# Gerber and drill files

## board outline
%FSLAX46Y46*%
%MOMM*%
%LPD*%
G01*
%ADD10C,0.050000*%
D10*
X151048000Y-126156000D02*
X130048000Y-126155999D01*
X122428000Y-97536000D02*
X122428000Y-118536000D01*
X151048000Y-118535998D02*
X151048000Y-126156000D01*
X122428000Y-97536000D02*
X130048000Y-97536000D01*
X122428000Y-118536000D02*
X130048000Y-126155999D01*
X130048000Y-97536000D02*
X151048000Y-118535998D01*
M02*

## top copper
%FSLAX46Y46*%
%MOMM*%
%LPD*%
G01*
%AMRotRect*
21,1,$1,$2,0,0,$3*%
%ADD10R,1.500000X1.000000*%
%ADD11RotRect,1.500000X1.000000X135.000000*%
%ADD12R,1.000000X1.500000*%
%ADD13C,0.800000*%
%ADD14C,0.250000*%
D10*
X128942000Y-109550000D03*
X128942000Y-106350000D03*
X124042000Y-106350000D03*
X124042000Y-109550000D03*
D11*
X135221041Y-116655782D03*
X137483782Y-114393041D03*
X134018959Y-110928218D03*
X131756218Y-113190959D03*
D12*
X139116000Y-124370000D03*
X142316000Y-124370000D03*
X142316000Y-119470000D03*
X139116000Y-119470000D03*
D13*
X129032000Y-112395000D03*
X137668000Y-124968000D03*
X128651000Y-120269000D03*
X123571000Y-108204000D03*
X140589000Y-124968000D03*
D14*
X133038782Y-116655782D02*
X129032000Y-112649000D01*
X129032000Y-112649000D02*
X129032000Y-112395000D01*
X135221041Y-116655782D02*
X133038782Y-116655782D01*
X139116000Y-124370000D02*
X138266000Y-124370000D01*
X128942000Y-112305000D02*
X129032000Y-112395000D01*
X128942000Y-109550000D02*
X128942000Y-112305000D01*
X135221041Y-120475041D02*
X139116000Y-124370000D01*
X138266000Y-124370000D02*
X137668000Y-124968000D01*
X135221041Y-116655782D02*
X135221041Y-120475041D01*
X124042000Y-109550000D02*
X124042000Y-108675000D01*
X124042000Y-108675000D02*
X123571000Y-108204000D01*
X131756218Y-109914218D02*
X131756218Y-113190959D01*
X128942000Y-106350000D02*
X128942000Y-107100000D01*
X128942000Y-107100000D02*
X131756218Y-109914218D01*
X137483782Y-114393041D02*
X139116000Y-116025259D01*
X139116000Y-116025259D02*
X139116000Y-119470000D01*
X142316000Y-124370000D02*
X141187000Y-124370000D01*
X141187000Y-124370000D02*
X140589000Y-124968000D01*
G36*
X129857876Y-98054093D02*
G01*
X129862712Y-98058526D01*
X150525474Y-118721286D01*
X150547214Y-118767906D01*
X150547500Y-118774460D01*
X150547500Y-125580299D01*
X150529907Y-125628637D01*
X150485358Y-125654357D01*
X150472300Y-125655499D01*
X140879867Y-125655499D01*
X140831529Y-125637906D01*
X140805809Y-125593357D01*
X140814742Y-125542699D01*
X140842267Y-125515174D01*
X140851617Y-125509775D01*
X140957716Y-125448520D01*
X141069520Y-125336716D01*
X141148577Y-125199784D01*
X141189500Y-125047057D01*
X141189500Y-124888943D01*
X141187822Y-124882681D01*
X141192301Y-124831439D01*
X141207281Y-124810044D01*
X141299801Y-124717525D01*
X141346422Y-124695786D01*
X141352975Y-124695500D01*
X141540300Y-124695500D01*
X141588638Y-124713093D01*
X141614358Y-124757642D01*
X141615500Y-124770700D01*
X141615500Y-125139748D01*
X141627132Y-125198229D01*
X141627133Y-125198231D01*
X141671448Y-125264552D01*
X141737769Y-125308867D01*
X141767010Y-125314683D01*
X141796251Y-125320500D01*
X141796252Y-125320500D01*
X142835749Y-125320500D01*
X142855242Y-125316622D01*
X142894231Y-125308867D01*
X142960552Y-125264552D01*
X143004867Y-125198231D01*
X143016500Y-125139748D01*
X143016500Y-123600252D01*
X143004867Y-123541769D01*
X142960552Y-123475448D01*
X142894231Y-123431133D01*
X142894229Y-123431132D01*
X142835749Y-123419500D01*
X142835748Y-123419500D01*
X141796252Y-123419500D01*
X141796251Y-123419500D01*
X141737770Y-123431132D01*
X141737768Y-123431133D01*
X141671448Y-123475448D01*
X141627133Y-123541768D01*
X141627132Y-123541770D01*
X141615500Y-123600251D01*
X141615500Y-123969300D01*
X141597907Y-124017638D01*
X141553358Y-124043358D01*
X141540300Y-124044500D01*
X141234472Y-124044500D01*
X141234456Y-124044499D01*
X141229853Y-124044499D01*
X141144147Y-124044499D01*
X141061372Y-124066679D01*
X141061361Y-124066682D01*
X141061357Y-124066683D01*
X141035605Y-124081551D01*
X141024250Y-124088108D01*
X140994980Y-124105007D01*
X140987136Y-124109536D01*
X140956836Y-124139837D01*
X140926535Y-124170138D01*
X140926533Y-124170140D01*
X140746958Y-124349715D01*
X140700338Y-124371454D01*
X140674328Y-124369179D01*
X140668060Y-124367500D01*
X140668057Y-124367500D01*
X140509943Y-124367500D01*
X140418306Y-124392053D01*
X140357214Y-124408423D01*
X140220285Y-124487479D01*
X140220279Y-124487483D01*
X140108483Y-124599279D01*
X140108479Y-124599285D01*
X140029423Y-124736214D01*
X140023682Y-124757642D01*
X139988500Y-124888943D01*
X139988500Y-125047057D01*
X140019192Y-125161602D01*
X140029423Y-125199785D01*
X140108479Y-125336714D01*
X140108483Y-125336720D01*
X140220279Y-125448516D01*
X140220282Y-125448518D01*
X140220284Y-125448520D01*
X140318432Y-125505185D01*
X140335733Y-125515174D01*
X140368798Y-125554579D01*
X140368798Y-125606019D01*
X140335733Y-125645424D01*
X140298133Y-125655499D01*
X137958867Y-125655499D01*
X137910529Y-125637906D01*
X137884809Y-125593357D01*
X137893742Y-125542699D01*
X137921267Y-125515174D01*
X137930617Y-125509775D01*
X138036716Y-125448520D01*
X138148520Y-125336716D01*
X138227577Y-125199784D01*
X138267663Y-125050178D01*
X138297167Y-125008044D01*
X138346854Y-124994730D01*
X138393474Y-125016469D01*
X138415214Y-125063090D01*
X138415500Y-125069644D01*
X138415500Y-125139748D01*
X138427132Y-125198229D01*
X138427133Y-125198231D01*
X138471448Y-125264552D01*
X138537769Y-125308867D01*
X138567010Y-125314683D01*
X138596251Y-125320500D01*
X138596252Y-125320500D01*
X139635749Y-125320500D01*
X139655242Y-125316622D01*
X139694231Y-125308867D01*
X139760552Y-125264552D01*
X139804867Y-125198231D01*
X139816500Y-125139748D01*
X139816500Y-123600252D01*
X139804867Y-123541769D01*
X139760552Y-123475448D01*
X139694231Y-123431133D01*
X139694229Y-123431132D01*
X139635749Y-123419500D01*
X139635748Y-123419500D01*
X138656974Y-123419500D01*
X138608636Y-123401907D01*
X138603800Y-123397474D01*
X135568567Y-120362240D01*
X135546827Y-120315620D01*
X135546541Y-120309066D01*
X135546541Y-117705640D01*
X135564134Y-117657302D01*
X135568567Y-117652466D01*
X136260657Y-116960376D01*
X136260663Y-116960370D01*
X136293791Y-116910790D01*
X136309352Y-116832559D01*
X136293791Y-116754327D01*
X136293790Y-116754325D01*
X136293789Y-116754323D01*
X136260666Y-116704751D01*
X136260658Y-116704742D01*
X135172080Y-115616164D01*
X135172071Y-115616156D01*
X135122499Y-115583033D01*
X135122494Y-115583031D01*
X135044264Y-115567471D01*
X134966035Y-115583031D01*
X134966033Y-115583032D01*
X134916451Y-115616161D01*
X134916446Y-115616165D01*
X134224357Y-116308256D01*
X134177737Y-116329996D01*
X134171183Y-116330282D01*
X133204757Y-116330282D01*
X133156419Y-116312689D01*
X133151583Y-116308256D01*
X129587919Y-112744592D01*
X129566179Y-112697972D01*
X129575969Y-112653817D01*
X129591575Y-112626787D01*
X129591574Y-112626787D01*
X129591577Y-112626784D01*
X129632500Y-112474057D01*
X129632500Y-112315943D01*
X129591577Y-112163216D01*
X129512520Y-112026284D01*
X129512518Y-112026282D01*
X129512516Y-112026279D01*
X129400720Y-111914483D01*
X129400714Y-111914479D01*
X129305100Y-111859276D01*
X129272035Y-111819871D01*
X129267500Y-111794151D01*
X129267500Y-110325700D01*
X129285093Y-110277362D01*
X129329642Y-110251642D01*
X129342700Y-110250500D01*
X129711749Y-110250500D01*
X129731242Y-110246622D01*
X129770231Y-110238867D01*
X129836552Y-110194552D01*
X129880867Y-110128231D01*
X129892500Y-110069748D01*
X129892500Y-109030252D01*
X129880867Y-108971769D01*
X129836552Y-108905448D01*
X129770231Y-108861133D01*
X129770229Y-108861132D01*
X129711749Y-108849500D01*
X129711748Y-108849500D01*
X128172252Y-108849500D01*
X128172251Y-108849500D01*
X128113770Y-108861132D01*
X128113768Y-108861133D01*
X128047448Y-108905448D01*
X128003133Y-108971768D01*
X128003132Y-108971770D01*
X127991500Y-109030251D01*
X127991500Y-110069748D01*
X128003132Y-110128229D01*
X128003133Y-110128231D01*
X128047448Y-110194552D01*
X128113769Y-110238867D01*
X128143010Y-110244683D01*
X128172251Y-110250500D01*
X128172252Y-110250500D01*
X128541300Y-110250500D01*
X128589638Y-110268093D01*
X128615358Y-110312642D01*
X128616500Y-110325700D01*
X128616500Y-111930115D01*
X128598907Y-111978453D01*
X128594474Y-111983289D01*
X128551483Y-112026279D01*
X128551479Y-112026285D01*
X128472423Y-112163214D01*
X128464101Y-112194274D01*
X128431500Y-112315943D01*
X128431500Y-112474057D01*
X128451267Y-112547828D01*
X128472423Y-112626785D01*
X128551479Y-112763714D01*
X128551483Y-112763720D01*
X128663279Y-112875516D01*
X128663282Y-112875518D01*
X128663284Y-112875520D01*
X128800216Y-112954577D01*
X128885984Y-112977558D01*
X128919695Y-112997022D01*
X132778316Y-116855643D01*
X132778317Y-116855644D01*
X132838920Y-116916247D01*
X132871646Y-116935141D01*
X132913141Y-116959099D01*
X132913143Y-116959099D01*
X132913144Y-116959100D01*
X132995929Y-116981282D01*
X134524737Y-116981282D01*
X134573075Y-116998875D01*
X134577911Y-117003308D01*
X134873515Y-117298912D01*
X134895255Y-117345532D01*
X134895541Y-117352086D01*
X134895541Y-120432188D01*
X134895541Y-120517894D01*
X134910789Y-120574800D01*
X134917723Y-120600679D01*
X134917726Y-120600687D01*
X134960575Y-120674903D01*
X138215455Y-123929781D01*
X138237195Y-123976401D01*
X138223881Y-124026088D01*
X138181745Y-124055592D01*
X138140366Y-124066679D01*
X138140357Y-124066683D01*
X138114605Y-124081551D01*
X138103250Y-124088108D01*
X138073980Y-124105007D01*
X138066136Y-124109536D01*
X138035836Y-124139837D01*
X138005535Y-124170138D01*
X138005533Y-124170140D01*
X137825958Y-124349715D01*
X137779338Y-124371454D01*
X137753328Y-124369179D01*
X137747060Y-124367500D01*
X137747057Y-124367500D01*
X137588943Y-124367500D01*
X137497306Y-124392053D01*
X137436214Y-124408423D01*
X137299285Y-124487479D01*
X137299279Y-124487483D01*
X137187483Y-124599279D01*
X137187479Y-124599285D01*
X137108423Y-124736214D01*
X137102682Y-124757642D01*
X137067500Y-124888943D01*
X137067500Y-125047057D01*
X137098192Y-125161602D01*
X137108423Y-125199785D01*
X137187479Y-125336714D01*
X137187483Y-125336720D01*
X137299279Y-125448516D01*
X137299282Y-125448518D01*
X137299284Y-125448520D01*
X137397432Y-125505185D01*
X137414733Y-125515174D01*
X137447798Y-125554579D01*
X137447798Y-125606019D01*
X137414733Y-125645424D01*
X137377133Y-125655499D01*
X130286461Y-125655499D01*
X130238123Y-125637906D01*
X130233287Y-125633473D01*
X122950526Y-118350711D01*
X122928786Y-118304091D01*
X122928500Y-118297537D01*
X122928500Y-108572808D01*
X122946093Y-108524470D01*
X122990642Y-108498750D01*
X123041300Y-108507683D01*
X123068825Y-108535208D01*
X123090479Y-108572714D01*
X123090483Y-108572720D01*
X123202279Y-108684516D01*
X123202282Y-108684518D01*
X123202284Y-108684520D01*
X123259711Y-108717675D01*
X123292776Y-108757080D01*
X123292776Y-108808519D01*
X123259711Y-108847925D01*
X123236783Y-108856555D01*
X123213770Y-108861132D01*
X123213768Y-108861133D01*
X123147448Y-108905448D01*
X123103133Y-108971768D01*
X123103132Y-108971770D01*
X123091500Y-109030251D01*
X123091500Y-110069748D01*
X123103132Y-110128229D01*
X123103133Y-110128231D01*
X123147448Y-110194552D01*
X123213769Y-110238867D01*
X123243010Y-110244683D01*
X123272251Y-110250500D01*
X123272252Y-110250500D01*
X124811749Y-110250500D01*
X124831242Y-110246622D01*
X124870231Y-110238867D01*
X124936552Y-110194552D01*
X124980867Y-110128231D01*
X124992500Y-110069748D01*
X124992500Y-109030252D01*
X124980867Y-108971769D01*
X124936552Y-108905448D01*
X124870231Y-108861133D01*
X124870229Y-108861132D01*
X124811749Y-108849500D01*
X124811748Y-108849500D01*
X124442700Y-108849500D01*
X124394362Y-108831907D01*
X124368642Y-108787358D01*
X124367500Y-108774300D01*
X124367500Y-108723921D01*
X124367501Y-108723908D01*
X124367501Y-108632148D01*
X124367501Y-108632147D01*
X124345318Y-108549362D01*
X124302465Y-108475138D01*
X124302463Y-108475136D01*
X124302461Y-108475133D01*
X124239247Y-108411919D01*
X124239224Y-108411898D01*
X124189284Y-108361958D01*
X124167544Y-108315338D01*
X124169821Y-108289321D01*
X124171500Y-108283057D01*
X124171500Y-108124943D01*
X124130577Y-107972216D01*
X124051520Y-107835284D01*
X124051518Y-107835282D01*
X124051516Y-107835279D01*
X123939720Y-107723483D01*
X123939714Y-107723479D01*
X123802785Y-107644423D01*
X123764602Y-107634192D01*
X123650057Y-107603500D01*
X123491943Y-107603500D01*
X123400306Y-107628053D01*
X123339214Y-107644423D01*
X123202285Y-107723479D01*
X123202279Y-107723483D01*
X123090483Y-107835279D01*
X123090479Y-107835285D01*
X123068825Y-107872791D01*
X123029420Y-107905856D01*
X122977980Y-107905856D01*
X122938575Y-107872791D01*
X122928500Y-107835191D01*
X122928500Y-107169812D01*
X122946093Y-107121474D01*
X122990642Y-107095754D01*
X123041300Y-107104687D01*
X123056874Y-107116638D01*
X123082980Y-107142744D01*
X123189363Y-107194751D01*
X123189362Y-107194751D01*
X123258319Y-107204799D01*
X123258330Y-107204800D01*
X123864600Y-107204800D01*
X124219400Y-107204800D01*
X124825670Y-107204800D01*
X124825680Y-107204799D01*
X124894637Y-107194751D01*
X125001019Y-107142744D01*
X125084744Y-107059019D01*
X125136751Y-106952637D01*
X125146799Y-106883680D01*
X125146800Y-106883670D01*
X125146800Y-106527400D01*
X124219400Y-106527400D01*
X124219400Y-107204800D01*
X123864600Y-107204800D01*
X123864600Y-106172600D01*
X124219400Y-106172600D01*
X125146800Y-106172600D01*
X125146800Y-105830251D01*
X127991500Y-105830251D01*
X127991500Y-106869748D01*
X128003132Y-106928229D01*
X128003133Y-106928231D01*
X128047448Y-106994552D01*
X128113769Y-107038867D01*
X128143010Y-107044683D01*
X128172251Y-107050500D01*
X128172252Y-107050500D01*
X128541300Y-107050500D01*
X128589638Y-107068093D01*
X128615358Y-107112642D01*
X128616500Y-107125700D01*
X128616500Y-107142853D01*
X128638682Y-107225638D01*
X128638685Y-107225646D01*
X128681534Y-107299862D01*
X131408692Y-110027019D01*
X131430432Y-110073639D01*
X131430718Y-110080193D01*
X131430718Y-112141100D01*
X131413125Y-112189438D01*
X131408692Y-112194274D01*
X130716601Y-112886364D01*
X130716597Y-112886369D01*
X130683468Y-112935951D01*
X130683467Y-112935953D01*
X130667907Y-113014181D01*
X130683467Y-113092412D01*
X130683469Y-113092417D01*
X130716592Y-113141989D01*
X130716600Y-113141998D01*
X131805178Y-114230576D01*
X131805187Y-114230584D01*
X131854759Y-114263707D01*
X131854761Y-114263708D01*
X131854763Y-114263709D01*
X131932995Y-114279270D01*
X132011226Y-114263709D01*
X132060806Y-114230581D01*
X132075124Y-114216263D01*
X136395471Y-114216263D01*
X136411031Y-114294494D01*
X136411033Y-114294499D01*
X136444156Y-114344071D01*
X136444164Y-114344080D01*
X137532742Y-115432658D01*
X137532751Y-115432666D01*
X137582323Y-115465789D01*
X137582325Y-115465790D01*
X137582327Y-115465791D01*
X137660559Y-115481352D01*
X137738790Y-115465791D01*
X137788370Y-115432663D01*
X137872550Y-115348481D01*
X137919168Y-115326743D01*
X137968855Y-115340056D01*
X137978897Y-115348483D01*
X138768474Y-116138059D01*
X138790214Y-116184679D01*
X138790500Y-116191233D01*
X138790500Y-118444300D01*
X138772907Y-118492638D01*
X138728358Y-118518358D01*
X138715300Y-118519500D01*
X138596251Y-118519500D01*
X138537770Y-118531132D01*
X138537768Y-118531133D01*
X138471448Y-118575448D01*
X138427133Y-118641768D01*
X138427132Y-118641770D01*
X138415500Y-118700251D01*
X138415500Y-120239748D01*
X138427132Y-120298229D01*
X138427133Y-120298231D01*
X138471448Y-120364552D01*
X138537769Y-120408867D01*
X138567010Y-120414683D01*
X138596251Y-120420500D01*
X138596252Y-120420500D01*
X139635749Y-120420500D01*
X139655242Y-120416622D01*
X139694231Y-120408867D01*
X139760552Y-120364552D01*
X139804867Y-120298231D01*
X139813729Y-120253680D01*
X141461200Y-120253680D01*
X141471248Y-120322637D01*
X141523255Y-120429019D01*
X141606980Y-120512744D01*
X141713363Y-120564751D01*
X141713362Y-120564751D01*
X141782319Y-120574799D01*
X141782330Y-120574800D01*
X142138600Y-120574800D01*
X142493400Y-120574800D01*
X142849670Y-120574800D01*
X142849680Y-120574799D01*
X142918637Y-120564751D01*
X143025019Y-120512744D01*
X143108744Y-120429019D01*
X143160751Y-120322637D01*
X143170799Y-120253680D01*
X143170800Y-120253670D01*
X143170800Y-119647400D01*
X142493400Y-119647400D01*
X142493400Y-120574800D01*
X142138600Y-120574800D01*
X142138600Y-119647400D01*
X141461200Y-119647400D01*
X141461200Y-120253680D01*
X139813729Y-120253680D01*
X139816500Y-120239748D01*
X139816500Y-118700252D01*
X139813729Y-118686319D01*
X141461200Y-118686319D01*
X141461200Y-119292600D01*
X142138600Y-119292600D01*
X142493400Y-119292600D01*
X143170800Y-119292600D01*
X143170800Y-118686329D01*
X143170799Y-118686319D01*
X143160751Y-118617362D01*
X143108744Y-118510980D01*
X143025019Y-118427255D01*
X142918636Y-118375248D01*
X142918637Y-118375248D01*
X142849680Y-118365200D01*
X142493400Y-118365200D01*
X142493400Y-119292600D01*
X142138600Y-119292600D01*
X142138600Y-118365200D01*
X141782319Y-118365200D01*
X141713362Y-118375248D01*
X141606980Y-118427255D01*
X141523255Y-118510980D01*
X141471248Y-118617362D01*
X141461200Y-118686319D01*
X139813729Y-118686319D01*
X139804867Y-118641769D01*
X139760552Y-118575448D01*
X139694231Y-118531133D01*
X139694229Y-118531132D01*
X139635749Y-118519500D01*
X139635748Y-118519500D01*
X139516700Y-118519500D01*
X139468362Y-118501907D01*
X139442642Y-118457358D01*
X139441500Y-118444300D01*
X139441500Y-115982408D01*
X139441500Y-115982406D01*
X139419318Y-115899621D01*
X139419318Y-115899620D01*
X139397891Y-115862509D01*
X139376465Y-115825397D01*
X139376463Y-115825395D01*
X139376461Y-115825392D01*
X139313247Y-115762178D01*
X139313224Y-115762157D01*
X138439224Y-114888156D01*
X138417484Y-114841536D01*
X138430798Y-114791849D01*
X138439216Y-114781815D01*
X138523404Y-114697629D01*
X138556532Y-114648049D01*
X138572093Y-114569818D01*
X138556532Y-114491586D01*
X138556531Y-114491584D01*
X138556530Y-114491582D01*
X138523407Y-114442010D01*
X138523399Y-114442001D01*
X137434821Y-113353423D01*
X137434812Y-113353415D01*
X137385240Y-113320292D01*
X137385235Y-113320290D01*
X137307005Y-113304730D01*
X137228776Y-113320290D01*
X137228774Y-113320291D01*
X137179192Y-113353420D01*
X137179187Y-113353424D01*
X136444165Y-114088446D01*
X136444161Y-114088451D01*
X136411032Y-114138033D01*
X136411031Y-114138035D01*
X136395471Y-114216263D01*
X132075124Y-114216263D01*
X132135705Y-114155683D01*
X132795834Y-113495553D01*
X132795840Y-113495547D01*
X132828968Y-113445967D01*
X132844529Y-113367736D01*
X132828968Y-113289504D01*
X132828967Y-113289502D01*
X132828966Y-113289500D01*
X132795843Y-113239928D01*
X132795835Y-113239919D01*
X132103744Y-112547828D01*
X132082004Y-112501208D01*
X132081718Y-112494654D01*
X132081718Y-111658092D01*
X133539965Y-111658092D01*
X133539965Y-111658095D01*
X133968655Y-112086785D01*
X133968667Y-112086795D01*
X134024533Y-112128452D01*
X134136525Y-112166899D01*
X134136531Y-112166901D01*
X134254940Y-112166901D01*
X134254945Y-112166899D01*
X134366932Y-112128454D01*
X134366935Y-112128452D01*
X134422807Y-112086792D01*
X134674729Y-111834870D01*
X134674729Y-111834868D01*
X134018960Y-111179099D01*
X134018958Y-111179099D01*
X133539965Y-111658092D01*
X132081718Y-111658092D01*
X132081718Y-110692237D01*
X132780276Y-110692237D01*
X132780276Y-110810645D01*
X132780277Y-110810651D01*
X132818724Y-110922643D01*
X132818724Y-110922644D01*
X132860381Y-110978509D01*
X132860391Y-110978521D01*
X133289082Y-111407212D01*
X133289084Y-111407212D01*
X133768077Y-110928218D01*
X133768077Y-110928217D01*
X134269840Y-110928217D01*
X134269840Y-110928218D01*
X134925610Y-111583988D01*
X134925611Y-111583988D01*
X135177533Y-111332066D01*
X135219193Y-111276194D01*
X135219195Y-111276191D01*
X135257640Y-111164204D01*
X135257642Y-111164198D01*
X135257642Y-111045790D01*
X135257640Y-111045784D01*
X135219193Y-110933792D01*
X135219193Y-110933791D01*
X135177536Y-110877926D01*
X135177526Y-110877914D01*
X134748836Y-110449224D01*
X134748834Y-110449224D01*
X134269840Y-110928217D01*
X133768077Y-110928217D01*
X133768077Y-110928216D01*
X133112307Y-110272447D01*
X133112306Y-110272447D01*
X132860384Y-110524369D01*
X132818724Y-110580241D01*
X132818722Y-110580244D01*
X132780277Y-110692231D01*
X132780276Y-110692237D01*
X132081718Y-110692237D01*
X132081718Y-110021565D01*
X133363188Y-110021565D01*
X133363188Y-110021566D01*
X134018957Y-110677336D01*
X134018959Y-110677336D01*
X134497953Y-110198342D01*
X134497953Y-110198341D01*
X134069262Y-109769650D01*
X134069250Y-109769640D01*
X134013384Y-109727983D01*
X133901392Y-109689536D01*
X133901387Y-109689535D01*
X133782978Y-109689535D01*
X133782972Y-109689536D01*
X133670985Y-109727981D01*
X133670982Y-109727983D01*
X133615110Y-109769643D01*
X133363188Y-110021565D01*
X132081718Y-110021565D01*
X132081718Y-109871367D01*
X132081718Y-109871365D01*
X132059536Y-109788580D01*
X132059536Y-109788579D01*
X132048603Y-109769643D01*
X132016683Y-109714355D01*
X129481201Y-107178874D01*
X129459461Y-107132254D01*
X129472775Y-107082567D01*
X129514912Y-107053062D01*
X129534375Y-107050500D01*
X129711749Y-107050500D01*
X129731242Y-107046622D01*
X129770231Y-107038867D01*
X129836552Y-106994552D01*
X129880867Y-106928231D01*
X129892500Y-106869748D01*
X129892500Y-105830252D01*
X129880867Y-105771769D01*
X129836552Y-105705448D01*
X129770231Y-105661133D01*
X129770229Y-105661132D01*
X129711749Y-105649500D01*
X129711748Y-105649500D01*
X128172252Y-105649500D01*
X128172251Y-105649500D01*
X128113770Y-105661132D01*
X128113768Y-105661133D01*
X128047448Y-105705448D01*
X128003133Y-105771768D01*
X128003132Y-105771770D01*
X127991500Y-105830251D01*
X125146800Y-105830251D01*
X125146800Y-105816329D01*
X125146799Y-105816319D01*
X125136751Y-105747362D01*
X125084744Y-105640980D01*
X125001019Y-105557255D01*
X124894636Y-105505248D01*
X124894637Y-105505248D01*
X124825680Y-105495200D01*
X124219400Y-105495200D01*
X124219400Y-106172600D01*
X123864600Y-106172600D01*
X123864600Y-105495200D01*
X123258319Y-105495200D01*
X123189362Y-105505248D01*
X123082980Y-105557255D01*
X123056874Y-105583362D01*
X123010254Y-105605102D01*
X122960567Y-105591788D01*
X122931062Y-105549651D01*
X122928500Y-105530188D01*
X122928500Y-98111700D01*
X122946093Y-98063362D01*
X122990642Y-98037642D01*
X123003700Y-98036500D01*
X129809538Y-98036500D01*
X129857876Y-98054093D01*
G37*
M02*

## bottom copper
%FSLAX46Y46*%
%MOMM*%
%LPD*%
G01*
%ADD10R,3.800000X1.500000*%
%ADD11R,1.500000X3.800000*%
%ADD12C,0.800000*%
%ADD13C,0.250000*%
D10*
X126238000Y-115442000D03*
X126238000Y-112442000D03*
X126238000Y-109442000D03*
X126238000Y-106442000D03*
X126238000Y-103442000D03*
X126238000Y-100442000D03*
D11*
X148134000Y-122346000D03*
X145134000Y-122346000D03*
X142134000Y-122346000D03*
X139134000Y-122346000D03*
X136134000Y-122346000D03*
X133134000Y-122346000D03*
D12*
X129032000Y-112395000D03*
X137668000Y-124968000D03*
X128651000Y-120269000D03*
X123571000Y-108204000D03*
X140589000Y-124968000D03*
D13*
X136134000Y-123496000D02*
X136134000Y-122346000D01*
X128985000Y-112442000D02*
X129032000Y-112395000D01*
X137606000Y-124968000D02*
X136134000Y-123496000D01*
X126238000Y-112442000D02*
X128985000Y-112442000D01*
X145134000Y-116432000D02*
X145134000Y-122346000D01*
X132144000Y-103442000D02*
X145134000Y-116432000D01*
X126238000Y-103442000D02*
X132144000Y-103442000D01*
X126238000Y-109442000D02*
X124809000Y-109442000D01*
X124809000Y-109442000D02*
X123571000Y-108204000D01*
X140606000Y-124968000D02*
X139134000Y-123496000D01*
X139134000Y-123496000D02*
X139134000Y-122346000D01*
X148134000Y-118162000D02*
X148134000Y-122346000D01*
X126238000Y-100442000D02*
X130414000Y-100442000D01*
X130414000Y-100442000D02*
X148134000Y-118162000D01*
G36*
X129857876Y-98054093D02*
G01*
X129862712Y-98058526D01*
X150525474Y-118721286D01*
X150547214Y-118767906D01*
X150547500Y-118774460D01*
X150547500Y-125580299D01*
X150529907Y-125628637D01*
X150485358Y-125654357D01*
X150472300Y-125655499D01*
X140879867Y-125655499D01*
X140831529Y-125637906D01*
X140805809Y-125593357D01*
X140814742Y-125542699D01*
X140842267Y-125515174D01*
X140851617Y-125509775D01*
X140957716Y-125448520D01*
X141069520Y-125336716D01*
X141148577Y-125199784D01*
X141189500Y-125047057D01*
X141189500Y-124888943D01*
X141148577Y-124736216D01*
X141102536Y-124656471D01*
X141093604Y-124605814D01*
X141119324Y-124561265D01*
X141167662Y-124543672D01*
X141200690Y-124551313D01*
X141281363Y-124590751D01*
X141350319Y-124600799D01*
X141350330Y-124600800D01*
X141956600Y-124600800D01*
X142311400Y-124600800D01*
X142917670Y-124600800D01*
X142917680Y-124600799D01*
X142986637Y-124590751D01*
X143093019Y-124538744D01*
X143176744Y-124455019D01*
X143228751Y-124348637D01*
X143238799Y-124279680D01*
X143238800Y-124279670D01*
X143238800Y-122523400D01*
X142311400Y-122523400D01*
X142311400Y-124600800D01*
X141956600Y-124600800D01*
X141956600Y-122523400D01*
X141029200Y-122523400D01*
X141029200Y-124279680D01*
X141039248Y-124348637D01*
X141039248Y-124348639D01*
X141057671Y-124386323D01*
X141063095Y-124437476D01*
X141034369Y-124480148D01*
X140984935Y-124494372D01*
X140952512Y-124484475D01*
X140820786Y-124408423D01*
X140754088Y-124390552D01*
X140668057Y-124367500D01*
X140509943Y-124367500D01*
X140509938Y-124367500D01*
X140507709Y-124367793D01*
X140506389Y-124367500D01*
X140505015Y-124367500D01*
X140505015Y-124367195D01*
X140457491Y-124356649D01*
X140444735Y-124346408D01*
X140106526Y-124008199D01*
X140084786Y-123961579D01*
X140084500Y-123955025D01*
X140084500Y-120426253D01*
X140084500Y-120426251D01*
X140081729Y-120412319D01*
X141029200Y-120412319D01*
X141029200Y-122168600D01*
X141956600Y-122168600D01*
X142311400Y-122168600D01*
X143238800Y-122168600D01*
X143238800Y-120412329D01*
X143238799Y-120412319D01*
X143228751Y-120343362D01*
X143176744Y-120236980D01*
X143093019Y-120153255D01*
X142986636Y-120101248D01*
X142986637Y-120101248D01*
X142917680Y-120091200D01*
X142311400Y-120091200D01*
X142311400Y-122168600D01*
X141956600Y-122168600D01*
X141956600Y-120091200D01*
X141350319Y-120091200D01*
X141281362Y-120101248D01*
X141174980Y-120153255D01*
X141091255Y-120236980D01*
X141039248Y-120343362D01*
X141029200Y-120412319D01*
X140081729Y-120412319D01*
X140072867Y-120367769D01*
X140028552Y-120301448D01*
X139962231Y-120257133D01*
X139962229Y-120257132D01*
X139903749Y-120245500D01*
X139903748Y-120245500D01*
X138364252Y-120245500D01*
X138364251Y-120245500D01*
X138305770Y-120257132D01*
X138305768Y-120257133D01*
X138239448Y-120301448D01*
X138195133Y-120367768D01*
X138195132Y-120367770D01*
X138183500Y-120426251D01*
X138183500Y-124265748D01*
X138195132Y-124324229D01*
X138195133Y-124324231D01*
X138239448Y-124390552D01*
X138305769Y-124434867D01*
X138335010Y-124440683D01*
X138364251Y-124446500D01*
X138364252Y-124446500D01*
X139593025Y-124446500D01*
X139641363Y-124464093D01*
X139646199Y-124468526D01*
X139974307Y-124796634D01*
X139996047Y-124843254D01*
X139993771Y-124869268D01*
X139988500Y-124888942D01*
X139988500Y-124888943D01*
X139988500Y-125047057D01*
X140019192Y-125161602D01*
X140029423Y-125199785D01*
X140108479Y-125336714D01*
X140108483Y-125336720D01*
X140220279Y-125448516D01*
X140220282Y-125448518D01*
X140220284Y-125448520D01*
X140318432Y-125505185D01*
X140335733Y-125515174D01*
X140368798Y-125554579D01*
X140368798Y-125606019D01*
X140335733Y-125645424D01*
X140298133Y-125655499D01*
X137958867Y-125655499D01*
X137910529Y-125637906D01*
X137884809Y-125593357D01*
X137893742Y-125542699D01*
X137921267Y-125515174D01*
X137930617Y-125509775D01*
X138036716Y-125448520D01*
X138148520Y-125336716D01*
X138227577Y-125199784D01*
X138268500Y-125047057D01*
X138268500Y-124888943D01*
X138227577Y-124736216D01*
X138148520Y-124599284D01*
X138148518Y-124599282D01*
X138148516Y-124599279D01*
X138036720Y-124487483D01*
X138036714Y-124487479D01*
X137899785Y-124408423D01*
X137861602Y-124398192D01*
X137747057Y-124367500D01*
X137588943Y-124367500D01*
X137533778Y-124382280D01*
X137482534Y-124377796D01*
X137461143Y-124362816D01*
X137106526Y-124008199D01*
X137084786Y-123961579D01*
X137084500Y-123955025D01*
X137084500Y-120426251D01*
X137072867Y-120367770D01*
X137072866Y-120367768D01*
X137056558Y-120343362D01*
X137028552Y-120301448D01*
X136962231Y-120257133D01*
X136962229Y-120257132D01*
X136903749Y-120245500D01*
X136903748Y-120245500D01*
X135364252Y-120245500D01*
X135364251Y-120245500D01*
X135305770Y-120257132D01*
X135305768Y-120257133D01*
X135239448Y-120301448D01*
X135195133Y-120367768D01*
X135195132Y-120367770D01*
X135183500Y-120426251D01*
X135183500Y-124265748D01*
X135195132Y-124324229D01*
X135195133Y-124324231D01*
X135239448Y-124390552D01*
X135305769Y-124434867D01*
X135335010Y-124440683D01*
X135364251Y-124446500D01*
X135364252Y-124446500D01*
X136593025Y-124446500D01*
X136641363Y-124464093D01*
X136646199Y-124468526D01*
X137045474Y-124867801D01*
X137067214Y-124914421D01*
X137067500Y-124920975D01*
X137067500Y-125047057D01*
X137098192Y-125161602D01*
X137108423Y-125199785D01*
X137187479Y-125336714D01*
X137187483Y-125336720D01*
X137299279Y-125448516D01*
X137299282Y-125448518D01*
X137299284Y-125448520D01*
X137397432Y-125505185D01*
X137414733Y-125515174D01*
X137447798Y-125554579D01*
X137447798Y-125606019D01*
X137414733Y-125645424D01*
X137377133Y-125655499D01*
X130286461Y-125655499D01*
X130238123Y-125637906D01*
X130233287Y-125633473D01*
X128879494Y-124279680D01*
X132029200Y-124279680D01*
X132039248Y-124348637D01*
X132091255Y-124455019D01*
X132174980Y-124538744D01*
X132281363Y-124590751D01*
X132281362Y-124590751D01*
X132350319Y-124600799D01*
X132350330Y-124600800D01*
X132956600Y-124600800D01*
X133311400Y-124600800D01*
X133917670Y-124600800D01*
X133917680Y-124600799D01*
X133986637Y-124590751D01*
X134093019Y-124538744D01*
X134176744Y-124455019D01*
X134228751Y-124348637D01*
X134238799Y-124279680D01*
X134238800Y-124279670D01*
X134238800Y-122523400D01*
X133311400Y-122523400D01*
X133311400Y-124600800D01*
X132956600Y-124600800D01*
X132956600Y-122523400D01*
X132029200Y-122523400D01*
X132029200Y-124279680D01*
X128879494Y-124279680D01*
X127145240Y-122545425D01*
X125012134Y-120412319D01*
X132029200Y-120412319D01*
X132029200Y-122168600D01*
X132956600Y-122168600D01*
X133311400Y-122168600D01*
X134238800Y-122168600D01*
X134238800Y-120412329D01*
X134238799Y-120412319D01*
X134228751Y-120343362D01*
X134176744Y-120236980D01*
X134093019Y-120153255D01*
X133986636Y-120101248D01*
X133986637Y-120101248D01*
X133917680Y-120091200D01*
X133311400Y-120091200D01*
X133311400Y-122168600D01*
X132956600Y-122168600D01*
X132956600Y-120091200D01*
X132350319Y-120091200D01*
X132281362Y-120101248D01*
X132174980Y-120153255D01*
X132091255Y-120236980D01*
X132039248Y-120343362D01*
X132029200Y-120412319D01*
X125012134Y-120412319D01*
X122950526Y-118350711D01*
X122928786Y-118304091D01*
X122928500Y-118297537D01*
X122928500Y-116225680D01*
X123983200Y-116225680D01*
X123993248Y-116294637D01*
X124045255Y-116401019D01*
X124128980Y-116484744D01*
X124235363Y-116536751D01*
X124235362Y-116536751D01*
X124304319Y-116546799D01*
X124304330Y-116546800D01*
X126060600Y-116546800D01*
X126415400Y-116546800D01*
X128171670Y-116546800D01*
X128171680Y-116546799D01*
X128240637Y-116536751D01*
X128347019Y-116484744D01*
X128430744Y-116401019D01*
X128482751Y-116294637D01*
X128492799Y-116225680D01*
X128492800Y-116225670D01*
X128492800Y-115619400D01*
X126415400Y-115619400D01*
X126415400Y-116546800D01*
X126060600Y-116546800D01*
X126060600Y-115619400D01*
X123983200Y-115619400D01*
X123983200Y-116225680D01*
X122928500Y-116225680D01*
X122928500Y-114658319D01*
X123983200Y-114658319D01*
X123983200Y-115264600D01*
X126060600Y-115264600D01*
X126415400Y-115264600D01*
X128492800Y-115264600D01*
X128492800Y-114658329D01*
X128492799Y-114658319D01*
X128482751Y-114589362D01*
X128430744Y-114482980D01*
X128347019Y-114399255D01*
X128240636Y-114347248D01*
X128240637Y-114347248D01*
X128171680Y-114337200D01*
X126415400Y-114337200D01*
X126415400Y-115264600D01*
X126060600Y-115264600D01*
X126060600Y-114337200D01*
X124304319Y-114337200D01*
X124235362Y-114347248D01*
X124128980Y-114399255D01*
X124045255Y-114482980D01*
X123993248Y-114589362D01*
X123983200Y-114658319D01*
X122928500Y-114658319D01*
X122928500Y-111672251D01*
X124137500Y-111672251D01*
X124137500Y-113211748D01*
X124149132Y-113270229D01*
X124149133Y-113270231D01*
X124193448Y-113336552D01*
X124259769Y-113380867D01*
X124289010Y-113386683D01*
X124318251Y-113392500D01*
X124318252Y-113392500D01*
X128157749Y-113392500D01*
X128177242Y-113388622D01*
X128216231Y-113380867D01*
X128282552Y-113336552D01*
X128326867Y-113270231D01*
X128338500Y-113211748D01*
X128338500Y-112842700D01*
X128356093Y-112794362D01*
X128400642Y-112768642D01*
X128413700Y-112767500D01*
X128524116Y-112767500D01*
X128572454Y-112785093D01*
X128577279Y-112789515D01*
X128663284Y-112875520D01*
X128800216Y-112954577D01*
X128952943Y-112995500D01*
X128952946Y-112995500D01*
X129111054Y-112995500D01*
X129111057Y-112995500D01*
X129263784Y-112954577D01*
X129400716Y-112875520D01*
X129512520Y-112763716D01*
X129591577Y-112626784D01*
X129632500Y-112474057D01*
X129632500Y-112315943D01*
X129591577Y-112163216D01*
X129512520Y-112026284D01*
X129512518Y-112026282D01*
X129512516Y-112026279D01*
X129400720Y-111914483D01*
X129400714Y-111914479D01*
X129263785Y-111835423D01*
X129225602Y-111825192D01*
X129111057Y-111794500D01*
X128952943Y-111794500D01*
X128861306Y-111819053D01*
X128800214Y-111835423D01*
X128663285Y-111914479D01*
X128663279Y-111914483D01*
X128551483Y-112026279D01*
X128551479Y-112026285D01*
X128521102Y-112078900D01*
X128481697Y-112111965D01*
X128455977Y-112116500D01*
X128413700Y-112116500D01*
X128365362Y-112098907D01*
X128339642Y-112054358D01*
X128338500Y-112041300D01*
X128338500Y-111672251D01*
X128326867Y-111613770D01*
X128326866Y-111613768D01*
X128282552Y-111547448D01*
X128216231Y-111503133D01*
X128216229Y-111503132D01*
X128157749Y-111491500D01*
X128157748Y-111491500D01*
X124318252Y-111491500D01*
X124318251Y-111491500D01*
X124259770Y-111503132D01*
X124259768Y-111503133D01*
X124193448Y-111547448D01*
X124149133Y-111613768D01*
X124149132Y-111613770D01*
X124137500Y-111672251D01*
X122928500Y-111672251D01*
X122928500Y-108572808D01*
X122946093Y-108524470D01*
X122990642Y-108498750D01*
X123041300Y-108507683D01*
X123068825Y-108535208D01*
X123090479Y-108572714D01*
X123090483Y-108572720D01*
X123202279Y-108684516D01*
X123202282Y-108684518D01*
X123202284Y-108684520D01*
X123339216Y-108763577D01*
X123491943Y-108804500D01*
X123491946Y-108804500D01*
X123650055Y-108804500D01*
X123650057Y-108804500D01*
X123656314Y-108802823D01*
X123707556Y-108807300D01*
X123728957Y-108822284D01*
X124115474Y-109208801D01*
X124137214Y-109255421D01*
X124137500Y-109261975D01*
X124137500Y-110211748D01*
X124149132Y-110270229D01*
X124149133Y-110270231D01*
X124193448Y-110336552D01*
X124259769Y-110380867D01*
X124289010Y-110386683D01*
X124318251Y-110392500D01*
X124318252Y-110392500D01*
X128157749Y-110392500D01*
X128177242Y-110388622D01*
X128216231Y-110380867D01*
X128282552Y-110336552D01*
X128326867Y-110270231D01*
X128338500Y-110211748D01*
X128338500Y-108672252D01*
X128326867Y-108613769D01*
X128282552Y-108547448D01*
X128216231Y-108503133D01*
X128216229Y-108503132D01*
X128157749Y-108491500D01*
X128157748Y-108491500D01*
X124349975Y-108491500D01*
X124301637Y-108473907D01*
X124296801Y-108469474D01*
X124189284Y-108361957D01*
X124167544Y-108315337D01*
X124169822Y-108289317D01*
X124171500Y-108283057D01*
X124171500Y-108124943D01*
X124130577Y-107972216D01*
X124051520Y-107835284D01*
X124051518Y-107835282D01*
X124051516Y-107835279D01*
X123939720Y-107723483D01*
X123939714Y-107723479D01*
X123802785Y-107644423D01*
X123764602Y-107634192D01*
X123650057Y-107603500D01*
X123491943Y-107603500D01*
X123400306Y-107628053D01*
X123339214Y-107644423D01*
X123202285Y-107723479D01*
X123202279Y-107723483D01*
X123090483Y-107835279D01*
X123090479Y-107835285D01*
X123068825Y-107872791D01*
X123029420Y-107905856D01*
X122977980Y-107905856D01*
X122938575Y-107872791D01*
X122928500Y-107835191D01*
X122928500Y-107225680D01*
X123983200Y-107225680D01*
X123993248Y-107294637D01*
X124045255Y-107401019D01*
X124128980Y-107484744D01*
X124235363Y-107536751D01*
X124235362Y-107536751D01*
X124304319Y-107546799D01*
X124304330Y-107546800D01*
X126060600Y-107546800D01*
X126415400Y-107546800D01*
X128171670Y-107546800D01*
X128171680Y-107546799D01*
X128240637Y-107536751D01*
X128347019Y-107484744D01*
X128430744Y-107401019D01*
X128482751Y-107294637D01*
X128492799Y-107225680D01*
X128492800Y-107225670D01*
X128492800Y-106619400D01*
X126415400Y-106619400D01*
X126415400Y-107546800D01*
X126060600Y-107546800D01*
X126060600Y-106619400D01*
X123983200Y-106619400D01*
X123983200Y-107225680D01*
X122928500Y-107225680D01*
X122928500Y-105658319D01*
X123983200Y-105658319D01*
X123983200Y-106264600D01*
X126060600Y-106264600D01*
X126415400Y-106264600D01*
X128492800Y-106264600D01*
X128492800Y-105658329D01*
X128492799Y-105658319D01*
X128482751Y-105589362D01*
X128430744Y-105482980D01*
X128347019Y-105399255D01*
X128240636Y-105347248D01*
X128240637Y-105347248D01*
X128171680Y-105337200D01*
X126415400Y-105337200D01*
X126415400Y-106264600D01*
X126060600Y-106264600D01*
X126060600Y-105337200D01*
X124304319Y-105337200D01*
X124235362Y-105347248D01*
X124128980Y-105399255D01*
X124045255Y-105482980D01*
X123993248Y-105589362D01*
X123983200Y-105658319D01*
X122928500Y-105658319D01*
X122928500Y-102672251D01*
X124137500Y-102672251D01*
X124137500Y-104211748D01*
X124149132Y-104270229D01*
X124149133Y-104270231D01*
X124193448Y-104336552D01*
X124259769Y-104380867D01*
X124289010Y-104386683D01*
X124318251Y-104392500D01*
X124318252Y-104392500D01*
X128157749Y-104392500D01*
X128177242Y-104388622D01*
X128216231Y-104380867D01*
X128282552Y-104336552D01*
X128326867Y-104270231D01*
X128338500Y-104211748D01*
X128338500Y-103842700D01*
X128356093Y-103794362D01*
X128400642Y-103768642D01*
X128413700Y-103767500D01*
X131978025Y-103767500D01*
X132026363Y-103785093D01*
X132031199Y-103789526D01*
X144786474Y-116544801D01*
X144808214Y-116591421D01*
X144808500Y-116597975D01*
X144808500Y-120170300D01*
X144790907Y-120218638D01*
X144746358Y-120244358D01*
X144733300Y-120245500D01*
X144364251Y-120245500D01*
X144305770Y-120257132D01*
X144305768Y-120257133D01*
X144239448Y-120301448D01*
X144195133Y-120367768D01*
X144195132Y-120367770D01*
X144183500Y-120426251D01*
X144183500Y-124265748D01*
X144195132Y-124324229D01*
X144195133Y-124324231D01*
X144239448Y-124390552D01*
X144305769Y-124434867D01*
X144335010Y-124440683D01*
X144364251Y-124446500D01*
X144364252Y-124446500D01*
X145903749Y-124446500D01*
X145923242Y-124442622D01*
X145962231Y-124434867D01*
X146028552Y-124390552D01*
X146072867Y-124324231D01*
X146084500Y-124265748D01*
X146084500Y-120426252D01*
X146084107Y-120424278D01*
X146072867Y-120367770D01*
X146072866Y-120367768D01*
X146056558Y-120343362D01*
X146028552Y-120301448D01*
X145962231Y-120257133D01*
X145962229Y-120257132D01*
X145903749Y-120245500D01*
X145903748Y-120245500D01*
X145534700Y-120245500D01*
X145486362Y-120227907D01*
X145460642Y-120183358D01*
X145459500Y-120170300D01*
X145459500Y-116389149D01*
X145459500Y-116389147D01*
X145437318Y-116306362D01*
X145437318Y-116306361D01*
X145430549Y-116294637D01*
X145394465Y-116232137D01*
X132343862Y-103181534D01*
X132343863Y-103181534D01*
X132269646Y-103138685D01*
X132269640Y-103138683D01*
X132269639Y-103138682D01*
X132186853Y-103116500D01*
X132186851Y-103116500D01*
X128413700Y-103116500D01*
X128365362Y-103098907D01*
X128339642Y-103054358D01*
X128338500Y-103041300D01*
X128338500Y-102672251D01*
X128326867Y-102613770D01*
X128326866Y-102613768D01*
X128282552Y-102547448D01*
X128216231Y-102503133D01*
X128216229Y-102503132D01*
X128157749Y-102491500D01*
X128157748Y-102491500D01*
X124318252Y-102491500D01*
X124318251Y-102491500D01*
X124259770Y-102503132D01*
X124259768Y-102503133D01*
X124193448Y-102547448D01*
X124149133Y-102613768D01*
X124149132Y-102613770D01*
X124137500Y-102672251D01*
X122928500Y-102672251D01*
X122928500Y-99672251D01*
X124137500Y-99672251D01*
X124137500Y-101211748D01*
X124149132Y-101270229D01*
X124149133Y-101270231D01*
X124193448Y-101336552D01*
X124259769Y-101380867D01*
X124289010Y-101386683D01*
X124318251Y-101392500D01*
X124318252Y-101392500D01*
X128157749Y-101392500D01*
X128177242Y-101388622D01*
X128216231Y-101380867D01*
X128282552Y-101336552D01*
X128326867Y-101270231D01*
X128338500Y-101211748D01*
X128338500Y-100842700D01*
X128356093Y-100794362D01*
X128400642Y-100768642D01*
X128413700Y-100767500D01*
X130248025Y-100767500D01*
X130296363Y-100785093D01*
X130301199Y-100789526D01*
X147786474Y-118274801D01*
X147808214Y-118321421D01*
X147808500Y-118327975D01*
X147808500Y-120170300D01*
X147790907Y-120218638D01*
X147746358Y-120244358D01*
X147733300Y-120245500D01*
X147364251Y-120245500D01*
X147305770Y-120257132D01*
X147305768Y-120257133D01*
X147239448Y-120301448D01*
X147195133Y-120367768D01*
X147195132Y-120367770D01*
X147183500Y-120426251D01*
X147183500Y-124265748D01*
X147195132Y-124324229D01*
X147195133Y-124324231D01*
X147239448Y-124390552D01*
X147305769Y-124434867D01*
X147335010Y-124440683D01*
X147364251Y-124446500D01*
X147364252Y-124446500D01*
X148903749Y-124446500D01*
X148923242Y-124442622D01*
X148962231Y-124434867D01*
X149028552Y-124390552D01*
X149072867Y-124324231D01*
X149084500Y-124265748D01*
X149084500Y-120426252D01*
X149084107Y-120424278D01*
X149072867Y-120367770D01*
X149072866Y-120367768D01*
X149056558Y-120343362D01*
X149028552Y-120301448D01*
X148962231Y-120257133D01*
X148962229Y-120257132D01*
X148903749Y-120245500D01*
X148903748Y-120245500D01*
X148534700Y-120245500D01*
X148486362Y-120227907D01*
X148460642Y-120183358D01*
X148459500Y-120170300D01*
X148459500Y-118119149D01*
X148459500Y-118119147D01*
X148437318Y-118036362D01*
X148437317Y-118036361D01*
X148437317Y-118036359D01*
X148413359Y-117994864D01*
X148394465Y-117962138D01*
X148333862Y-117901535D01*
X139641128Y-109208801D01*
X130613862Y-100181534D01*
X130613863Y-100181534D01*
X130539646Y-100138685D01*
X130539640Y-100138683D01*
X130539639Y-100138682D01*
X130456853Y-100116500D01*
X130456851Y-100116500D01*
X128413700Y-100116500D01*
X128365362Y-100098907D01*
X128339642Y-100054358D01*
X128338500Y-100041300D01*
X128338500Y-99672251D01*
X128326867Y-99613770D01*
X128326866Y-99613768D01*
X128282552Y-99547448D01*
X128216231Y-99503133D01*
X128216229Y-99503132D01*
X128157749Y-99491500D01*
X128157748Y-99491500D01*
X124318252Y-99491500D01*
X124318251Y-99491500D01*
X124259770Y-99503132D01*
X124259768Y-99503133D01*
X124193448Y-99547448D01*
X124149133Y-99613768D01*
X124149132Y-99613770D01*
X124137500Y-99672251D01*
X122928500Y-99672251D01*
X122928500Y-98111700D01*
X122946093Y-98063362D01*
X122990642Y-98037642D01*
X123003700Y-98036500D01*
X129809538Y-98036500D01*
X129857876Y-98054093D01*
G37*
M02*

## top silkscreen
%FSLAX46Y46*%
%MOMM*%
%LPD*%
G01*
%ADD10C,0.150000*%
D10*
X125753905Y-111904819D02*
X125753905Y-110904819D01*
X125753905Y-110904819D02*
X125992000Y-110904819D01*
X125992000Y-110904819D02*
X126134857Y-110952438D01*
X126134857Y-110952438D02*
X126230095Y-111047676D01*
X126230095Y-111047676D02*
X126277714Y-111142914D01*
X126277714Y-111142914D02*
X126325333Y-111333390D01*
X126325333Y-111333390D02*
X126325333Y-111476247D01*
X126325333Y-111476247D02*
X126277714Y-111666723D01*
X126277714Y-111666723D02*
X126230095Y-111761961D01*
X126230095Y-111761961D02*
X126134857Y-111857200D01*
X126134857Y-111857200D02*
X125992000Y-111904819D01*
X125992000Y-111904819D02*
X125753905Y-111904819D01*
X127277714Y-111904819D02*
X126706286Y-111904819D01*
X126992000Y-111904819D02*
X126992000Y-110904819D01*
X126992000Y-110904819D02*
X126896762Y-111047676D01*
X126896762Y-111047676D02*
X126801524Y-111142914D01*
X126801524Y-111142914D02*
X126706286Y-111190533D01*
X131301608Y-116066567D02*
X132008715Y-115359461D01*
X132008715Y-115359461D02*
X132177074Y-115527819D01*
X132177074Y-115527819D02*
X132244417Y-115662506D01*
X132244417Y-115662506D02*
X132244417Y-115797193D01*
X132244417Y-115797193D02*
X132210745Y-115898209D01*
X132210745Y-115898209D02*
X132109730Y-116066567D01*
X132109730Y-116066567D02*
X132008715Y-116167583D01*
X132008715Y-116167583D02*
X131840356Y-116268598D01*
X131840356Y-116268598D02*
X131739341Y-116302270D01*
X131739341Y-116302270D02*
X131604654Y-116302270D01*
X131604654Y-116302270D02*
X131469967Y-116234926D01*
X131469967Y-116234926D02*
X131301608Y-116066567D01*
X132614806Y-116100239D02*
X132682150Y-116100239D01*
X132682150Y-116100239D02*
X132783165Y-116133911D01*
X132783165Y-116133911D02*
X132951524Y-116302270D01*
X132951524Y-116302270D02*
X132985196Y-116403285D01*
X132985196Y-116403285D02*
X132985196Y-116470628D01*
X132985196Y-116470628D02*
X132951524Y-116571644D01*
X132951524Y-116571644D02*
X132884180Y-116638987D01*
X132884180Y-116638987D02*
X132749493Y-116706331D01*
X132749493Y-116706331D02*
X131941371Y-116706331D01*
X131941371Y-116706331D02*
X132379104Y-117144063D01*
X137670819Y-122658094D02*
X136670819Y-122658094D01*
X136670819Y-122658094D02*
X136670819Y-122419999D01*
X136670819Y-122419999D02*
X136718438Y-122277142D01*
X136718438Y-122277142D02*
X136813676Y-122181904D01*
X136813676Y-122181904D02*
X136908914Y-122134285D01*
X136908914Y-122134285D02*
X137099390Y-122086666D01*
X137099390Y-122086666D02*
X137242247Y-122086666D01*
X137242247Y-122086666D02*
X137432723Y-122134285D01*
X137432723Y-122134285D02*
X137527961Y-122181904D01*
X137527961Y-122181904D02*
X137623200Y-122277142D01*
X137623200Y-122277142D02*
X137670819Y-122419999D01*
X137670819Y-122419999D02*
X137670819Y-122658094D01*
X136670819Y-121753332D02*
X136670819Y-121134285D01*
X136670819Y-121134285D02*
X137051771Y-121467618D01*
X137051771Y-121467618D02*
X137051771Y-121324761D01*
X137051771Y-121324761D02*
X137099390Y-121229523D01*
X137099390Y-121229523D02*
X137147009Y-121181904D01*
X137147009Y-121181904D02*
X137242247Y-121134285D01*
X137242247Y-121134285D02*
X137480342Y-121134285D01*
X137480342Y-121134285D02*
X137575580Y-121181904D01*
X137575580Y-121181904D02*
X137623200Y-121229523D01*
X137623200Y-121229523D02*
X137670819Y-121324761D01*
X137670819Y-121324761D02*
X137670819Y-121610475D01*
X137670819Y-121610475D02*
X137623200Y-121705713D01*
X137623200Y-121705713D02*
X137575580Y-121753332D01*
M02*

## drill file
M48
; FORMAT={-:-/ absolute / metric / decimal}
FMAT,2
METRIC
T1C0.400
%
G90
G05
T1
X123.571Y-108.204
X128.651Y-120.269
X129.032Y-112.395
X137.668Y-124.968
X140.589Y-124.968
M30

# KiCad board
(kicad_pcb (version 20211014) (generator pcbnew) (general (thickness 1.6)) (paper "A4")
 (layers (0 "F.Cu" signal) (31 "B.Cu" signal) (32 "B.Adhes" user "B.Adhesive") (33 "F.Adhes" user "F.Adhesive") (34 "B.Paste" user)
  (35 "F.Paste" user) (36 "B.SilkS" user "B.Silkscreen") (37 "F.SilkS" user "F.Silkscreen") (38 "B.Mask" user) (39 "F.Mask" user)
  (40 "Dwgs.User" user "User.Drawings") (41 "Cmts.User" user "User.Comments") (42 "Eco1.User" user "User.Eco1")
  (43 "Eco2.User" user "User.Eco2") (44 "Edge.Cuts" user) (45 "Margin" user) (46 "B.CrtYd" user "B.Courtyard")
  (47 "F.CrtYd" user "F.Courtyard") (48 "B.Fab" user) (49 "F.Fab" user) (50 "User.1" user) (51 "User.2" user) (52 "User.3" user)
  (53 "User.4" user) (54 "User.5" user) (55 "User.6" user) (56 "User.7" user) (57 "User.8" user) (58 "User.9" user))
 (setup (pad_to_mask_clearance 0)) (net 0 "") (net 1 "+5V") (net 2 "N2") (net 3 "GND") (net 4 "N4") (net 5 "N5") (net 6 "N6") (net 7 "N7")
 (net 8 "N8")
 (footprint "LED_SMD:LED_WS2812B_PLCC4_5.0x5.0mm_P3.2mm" (layer "F.Cu") (at 126.492 107.95 180)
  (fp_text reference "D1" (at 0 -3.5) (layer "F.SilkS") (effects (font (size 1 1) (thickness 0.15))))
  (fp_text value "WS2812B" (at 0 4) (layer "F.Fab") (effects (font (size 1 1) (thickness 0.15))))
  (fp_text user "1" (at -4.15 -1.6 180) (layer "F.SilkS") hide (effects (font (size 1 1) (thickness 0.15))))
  (pad "1" smd rect (at -2.45 -1.6 180) (size 1.5 1) (layers "F.Cu" "F.Paste" "F.Mask") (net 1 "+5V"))
  (pad "2" smd rect (at -2.45 1.6 180) (size 1.5 1) (layers "F.Cu" "F.Paste" "F.Mask") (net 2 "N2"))
  (pad "3" smd rect (at 2.45 1.6 180) (size 1.5 1) (layers "F.Cu" "F.Paste" "F.Mask") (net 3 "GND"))
  (pad "4" smd rect (at 2.45 -1.6 180) (size 1.5 1) (layers "F.Cu" "F.Paste" "F.Mask") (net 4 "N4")))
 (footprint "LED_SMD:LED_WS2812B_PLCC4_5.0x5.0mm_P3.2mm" (layer "F.Cu") (at 134.62 113.792 135)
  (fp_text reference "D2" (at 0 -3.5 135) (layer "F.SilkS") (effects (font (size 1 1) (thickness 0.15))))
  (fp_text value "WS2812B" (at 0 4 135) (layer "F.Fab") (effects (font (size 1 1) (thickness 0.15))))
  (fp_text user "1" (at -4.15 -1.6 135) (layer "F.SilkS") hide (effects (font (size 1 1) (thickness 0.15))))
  (pad "1" smd rect (at -2.45 -1.6 135) (size 1.5 1) (layers "F.Cu" "F.Paste" "F.Mask") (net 1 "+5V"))
  (pad "2" smd rect (at -2.45 1.6 135) (size 1.5 1) (layers "F.Cu" "F.Paste" "F.Mask") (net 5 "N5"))
  (pad "3" smd rect (at 2.45 1.6 135) (size 1.5 1) (layers "F.Cu" "F.Paste" "F.Mask") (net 3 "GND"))
  (pad "4" smd rect (at 2.45 -1.6 135) (size 1.5 1) (layers "F.Cu" "F.Paste" "F.Mask") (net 2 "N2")))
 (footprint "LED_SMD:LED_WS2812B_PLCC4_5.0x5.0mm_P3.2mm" (layer "F.Cu") (at 140.716 121.92 90)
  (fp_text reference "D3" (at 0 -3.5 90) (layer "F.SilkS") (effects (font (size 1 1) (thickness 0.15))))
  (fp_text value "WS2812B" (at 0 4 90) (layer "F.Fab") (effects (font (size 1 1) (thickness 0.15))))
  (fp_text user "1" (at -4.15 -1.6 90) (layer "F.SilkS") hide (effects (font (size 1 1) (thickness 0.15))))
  (pad "1" smd rect (at -2.45 -1.6 90) (size 1.5 1) (layers "F.Cu" "F.Paste" "F.Mask") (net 1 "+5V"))
  (pad "2" smd rect (at -2.45 1.6 90) (size 1.5 1) (layers "F.Cu" "F.Paste" "F.Mask") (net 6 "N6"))
  (pad "3" smd rect (at 2.45 1.6 90) (size 1.5 1) (layers "F.Cu" "F.Paste" "F.Mask") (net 3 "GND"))
  (pad "4" smd rect (at 2.45 -1.6 90) (size 1.5 1) (layers "F.Cu" "F.Paste" "F.Mask") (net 5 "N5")))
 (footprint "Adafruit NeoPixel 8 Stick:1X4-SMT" (layer "B.Cu") (at 126.873 107.442 90)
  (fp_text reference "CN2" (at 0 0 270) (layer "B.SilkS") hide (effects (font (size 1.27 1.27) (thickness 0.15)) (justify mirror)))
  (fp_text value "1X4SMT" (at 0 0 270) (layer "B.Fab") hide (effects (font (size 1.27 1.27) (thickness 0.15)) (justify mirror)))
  (pad "1" smd rect (at -8 -0.635 90) (size 1.5 3.8) (layers "B.Cu" "B.Paste" "B.Mask") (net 3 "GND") (solder_mask_margin 0.1016))
  (pad "2" smd rect (at -5 -0.635 90) (size 1.5 3.8) (layers "B.Cu" "B.Paste" "B.Mask") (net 1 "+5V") (solder_mask_margin 0.1016))
  (pad "3" smd rect (at -2 -0.635 90) (size 1.5 3.8) (layers "B.Cu" "B.Paste" "B.Mask") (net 4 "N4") (solder_mask_margin 0.1016))
  (pad "4" smd rect (at 1 -0.635 90) (size 1.5 3.8) (layers "B.Cu" "B.Paste" "B.Mask") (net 3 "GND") (solder_mask_margin 0.1016))
  (pad "5" smd rect (at 4 -0.635 90) (size 1.5 3.8) (layers "B.Cu" "B.Paste" "B.Mask") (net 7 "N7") (solder_mask_margin 0.1016))
  (pad "6" smd rect (at 7 -0.635 90) (size 1.5 3.8) (layers "B.Cu" "B.Paste" "B.Mask") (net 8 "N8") (solder_mask_margin 0.1016)))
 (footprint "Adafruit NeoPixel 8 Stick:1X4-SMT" (layer "B.Cu") (at 140.134 121.711 180)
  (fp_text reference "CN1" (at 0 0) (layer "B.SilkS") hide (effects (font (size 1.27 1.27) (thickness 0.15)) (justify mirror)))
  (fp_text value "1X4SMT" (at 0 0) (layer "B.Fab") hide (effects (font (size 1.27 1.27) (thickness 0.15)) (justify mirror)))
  (pad "1" smd rect (at -8 -0.635 180) (size 1.5 3.8) (layers "B.Cu" "B.Paste" "B.Mask") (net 8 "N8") (solder_mask_margin 0.1016))
  (pad "2" smd rect (at -5 -0.635 180) (size 1.5 3.8) (layers "B.Cu" "B.Paste" "B.Mask") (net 7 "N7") (solder_mask_margin 0.1016))
  (pad "3" smd rect (at -2 -0.635 180) (size 1.5 3.8) (layers "B.Cu" "B.Paste" "B.Mask") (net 3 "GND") (solder_mask_margin 0.1016))
  (pad "4" smd rect (at 1 -0.635 180) (size 1.5 3.8) (layers "B.Cu" "B.Paste" "B.Mask") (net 6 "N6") (solder_mask_margin 0.1016))
  (pad "5" smd rect (at 4 -0.635 180) (size 1.5 3.8) (layers "B.Cu" "B.Paste" "B.Mask") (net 1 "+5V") (solder_mask_margin 0.1016))
  (pad "6" smd rect (at 7 -0.635 180) (size 1.5 3.8) (layers "B.Cu" "B.Paste" "B.Mask") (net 3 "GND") (solder_mask_margin 0.1016)))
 (gr_line (start 151.048 126.156) (end 130.048 126.155999) (layer "Edge.Cuts") (width 0.05))
 (gr_line (start 122.428 97.536) (end 122.428 118.536) (layer "Edge.Cuts") (width 0.05))
 (gr_line (start 151.048 118.535998) (end 151.048 126.156) (layer "Edge.Cuts") (width 0.05))
 (gr_line (start 122.428 97.536) (end 130.048 97.536) (layer "Edge.Cuts") (width 0.05))
 (gr_line (start 122.428 118.536) (end 130.048 126.155999) (layer "Edge.Cuts") (width 0.05))
 (gr_line (start 130.048 97.536) (end 151.048 118.535998) (layer "Edge.Cuts") (width 0.05))
 (segment (start 133.038782 116.655782) (end 129.032 112.649) (width 0.25) (layer "F.Cu") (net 1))
 (segment (start 129.032 112.649) (end 129.032 112.395) (width 0.25) (layer "F.Cu") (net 1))
 (segment (start 135.221041 116.655782) (end 133.038782 116.655782) (width 0.25) (layer "F.Cu") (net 1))
 (segment (start 139.116 124.37) (end 138.266 124.37) (width 0.25) (layer "F.Cu") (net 1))
 (segment (start 128.942 112.305) (end 129.032 112.395) (width 0.25) (layer "F.Cu") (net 1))
 (segment (start 128.942 109.55) (end 128.942 112.305) (width 0.25) (layer "F.Cu") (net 1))
 (segment (start 135.221041 120.475041) (end 139.116 124.37) (width 0.25) (layer "F.Cu") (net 1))
 (segment (start 138.266 124.37) (end 137.668 124.968) (width 0.25) (layer "F.Cu") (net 1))
 (segment (start 135.221041 116.655782) (end 135.221041 120.475041) (width 0.25) (layer "F.Cu") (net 1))
 (via (at 129.032 112.395) (size 0.8) (drill 0.4) (layers "F.Cu" "B.Cu") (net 1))
 (via (at 137.668 124.968) (size 0.8) (drill 0.4) (layers "F.Cu" "B.Cu") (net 1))
 (segment (start 136.134 123.496) (end 136.134 122.346) (width 0.25) (layer "B.Cu") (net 1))
 (segment (start 128.985 112.442) (end 129.032 112.395) (width 0.25) (layer "B.Cu") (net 1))
 (segment (start 137.606 124.968) (end 136.134 123.496) (width 0.25) (layer "B.Cu") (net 1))
 (segment (start 126.238 112.442) (end 128.985 112.442) (width 0.25) (layer "B.Cu") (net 1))
 (via (at 128.651 120.269) (size 0.8) (drill 0.4) (layers "F.Cu" "B.Cu") (free) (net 3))
 (segment (start 145.134 116.432) (end 145.134 122.346) (width 0.25) (layer "B.Cu") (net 7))
 (segment (start 132.144 103.442) (end 145.134 116.432) (width 0.25) (layer "B.Cu") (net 7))
 (segment (start 126.238 103.442) (end 132.144 103.442) (width 0.25) (layer "B.Cu") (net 7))
 (segment (start 124.042 109.55) (end 124.042 108.675) (width 0.25) (layer "F.Cu") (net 4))
 (segment (start 124.042 108.675) (end 123.571 108.204) (width 0.25) (layer "F.Cu") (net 4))
 (via (at 123.571 108.204) (size 0.8) (drill 0.4) (layers "F.Cu" "B.Cu") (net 4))
 (segment (start 126.238 109.442) (end 124.809 109.442) (width 0.25) (layer "B.Cu") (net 4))
 (segment (start 124.809 109.442) (end 123.571 108.204) (width 0.25) (layer "B.Cu") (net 4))
 (segment (start 131.756218 109.914218) (end 131.756218 113.190959) (width 0.25) (layer "F.Cu") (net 2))
 (segment (start 128.942 106.35) (end 128.942 107.1) (width 0.25) (layer "F.Cu") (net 2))
 (segment (start 128.942 107.1) (end 131.756218 109.914218) (width 0.25) (layer "F.Cu") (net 2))
 (segment (start 137.483782 114.393041) (end 139.116 116.025259) (width 0.25) (layer "F.Cu") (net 5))
 (segment (start 139.116 116.025259) (end 139.116 119.47) (width 0.25) (layer "F.Cu") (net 5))
 (segment (start 142.316 124.37) (end 141.187 124.37) (width 0.25) (layer "F.Cu") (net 6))
 (segment (start 141.187 124.37) (end 140.589 124.968) (width 0.25) (layer "F.Cu") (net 6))
 (via (at 140.589 124.968) (size 0.8) (drill 0.4) (layers "F.Cu" "B.Cu") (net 6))
 (segment (start 140.606 124.968) (end 139.134 123.496) (width 0.25) (layer "B.Cu") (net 6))
 (segment (start 139.134 123.496) (end 139.134 122.346) (width 0.25) (layer "B.Cu") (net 6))
 (segment (start 148.134 118.162) (end 148.134 122.346) (width 0.25) (layer "B.Cu") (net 8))
 (segment (start 126.238 100.442) (end 130.414 100.442) (width 0.25) (layer "B.Cu") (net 8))
 (segment (start 130.414 100.442) (end 148.134 118.162) (width 0.25) (layer "B.Cu") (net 8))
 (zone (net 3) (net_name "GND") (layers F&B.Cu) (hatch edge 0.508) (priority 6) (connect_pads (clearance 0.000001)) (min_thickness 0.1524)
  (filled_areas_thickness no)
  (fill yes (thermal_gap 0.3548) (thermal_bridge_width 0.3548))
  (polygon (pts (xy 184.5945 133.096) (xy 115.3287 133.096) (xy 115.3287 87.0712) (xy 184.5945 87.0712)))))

